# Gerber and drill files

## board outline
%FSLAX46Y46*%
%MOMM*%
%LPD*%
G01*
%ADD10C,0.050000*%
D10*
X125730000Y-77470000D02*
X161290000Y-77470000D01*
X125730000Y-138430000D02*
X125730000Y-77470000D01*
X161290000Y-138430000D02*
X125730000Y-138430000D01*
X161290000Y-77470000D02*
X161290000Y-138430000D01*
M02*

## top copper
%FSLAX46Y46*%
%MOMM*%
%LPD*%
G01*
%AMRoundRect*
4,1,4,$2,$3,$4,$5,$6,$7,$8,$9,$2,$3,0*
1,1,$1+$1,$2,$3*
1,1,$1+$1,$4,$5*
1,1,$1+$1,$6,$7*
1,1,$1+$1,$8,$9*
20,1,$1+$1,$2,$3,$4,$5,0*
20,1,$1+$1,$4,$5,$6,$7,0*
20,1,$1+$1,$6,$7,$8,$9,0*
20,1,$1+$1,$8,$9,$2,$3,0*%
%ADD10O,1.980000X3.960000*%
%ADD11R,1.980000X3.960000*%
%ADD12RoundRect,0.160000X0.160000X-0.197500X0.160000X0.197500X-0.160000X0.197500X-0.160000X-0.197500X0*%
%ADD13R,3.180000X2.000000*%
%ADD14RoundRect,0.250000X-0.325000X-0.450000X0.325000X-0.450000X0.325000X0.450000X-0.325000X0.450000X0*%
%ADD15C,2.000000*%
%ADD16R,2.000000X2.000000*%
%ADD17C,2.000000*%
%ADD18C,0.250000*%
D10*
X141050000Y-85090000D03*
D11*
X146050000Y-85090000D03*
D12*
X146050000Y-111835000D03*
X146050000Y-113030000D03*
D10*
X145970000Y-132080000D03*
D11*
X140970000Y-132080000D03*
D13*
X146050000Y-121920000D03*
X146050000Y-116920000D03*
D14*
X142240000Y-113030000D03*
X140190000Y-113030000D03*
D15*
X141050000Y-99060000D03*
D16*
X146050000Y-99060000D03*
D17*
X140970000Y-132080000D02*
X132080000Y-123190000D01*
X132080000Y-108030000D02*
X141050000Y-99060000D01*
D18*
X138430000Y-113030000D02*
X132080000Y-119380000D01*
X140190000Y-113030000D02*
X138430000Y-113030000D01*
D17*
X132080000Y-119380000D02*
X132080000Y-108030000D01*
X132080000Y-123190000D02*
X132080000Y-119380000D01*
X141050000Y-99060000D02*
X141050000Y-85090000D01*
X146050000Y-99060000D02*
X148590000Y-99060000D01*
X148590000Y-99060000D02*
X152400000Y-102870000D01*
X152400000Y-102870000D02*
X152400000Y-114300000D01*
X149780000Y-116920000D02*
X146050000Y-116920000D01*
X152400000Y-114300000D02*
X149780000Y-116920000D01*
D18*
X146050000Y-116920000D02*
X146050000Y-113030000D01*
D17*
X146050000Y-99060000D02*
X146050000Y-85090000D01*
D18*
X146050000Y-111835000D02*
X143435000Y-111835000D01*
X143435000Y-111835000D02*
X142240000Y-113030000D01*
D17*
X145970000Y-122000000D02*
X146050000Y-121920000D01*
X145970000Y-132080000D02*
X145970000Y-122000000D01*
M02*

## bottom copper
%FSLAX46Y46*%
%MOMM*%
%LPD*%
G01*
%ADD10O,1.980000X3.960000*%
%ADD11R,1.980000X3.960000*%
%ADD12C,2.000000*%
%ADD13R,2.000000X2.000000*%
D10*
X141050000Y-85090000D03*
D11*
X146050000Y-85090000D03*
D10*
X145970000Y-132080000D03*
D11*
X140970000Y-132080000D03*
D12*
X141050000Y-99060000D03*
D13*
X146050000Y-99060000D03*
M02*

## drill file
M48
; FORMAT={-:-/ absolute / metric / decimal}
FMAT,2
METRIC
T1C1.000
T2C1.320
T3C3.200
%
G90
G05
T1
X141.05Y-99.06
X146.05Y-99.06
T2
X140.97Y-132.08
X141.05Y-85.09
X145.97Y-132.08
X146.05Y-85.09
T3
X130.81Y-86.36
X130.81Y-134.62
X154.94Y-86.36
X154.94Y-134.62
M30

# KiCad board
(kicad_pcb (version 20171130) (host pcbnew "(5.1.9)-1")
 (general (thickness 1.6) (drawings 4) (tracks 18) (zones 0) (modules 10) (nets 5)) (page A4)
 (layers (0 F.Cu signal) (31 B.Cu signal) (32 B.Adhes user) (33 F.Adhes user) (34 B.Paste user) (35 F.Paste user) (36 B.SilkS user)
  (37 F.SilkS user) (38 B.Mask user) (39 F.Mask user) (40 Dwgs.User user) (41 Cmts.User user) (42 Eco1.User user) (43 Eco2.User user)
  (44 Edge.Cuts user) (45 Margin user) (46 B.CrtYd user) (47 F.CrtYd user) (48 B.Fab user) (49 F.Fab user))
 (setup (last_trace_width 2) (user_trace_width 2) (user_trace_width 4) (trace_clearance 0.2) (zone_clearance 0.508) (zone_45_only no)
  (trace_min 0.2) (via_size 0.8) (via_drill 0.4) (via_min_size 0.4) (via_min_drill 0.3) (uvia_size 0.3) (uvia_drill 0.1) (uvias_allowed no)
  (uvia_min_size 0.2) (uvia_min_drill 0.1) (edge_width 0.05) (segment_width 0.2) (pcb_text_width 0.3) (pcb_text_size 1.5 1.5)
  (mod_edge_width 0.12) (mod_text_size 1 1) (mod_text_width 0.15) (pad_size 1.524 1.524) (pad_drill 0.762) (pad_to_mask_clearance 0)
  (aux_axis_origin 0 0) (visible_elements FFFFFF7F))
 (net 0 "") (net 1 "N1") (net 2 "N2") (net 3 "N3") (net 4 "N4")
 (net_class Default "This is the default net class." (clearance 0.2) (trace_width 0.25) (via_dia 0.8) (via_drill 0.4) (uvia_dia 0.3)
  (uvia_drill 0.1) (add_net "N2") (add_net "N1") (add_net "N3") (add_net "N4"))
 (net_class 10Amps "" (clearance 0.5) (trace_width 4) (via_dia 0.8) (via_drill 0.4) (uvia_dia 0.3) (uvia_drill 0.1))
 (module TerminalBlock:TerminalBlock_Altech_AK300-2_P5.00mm (layer F.Cu) (at 146.05 85.09 180)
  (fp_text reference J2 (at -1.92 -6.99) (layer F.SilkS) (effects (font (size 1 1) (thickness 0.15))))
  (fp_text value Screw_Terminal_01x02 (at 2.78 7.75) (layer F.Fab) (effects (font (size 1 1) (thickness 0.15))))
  (pad 2 thru_hole oval (at 5 0 180) (size 1.98 3.96) (drill 1.32) (layers *.Cu *.Mask) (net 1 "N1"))
  (pad 1 thru_hole rect (at 0 0 180) (size 1.98 3.96) (drill 1.32) (layers *.Cu *.Mask) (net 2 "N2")))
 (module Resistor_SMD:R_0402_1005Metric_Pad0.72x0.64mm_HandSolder (layer F.Cu) (at 146.05 112.4325 90)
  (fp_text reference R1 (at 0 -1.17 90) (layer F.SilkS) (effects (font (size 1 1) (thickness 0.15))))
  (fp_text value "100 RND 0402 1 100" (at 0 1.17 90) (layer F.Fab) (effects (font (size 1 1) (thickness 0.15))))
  (pad 2 smd roundrect (at 0.5975 0 90) (size 0.715 0.64) (layers F.Cu F.Paste F.Mask) (roundrect_rratio 0.25) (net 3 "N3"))
  (pad 1 smd roundrect (at -0.5975 0 90) (size 0.715 0.64) (layers F.Cu F.Paste F.Mask) (roundrect_rratio 0.25) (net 2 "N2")))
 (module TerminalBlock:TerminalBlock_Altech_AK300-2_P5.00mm (layer F.Cu) (at 140.97 132.08)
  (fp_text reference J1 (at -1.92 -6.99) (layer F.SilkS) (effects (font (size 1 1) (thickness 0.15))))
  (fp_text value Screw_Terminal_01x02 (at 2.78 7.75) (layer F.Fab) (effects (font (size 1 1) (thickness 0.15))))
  (pad 2 thru_hole oval (at 5 0) (size 1.98 3.96) (drill 1.32) (layers *.Cu *.Mask) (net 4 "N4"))
  (pad 1 thru_hole rect (at 0 0) (size 1.98 3.96) (drill 1.32) (layers *.Cu *.Mask) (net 1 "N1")))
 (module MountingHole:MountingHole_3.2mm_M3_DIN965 (layer F.Cu) (at 154.94 134.62)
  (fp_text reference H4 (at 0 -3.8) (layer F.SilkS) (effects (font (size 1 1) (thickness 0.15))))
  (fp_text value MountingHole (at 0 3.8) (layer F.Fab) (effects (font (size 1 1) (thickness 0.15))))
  (pad 1 np_thru_hole circle (at 0 0) (size 3.2 3.2) (drill 3.2) (layers *.Cu *.Mask)))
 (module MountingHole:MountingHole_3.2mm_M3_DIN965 (layer F.Cu) (at 154.94 86.36)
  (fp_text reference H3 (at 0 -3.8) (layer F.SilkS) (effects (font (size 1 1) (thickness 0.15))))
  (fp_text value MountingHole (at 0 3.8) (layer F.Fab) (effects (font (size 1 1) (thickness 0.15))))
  (pad 1 np_thru_hole circle (at 0 0) (size 3.2 3.2) (drill 3.2) (layers *.Cu *.Mask)))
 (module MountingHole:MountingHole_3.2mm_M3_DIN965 (layer F.Cu) (at 130.81 86.36)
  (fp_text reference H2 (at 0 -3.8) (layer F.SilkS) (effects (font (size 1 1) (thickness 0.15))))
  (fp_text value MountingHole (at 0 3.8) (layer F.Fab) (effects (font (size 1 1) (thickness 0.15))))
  (pad 1 np_thru_hole circle (at 0 0) (size 3.2 3.2) (drill 3.2) (layers *.Cu *.Mask)))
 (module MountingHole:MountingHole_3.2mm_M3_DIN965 (layer F.Cu) (at 130.81 134.62)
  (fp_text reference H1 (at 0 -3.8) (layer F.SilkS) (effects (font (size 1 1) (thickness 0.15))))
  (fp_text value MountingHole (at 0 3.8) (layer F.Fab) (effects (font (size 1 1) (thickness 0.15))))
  (pad 1 np_thru_hole circle (at 0 0) (size 3.2 3.2) (drill 3.2) (layers *.Cu *.Mask)))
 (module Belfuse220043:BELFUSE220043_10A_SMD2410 (layer F.Cu) (at 149.86 119.42 270)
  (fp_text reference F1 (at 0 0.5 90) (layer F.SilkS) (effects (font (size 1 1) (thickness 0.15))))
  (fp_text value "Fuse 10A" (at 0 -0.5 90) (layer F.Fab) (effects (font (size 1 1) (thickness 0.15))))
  (pad 2 smd rect (at 2.5 3.81 270) (size 2 3.18) (layers F.Cu F.Paste F.Mask) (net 4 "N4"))
  (pad 1 smd rect (at -2.5 3.81 270) (size 2 3.18) (layers F.Cu F.Paste F.Mask) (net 2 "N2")))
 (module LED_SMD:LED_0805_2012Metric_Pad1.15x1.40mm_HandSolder (layer F.Cu) (at 141.215 113.03)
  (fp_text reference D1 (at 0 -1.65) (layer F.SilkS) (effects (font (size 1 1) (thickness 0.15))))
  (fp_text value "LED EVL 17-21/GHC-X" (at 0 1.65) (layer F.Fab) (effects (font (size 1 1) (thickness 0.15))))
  (pad 2 smd roundrect (at 1.025 0) (size 1.15 1.4) (layers F.Cu F.Paste F.Mask) (roundrect_rratio 0.217391) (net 3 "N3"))
  (pad 1 smd roundrect (at -1.025 0) (size 1.15 1.4) (layers F.Cu F.Paste F.Mask) (roundrect_rratio 0.217391) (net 1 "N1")))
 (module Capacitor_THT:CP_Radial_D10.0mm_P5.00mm (layer F.Cu) (at 146.05 99.06 180)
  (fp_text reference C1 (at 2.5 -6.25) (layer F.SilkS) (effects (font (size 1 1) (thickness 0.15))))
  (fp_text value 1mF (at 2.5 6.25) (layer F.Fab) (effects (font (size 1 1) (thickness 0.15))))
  (pad 2 thru_hole circle (at 5 0 180) (size 2 2) (drill 1) (layers *.Cu *.Mask) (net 1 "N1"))
  (pad 1 thru_hole rect (at 0 0 180) (size 2 2) (drill 1) (layers *.Cu *.Mask) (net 2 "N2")))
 (gr_line (start 125.73 77.47) (end 161.29 77.47) (layer Edge.Cuts) (width 0.05))
 (gr_line (start 125.73 138.43) (end 125.73 77.47) (layer Edge.Cuts) (width 0.05))
 (gr_line (start 161.29 138.43) (end 125.73 138.43) (layer Edge.Cuts) (width 0.05))
 (gr_line (start 161.29 77.47) (end 161.29 138.43) (layer Edge.Cuts) (width 0.05))
 (segment (start 140.97 132.08) (end 132.08 123.19) (width 2) (layer F.Cu) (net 1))
 (segment (start 132.08 108.03) (end 141.05 99.06) (width 2) (layer F.Cu) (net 1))
 (segment (start 138.43 113.03) (end 132.08 119.38) (width 0.25) (layer F.Cu) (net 1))
 (segment (start 140.19 113.03) (end 138.43 113.03) (width 0.25) (layer F.Cu) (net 1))
 (segment (start 132.08 119.38) (end 132.08 108.03) (width 2) (layer F.Cu) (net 1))
 (segment (start 132.08 123.19) (end 132.08 119.38) (width 2) (layer F.Cu) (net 1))
 (segment (start 141.05 99.06) (end 141.05 85.09) (width 2) (layer F.Cu) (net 1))
 (segment (start 146.05 99.06) (end 148.59 99.06) (width 2) (layer F.Cu) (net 2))
 (segment (start 148.59 99.06) (end 152.4 102.87) (width 2) (layer F.Cu) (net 2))
 (segment (start 152.4 102.87) (end 152.4 114.3) (width 2) (layer F.Cu) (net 2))
 (segment (start 149.78 116.92) (end 146.05 116.92) (width 2) (layer F.Cu) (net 2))
 (segment (start 152.4 114.3) (end 149.78 116.92) (width 2) (layer F.Cu) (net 2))
 (segment (start 146.05 116.92) (end 146.05 113.03) (width 0.25) (layer F.Cu) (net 2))
 (segment (start 146.05 99.06) (end 146.05 85.09) (width 2) (layer F.Cu) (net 2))
 (segment (start 146.05 111.835) (end 143.435 111.835) (width 0.25) (layer F.Cu) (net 3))
 (segment (start 143.435 111.835) (end 142.24 113.03) (width 0.25) (layer F.Cu) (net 3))
 (segment (start 145.97 122) (end 146.05 121.92) (width 2) (layer F.Cu) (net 4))
 (segment (start 145.97 132.08) (end 145.97 122) (width 2) (layer F.Cu) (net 4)))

